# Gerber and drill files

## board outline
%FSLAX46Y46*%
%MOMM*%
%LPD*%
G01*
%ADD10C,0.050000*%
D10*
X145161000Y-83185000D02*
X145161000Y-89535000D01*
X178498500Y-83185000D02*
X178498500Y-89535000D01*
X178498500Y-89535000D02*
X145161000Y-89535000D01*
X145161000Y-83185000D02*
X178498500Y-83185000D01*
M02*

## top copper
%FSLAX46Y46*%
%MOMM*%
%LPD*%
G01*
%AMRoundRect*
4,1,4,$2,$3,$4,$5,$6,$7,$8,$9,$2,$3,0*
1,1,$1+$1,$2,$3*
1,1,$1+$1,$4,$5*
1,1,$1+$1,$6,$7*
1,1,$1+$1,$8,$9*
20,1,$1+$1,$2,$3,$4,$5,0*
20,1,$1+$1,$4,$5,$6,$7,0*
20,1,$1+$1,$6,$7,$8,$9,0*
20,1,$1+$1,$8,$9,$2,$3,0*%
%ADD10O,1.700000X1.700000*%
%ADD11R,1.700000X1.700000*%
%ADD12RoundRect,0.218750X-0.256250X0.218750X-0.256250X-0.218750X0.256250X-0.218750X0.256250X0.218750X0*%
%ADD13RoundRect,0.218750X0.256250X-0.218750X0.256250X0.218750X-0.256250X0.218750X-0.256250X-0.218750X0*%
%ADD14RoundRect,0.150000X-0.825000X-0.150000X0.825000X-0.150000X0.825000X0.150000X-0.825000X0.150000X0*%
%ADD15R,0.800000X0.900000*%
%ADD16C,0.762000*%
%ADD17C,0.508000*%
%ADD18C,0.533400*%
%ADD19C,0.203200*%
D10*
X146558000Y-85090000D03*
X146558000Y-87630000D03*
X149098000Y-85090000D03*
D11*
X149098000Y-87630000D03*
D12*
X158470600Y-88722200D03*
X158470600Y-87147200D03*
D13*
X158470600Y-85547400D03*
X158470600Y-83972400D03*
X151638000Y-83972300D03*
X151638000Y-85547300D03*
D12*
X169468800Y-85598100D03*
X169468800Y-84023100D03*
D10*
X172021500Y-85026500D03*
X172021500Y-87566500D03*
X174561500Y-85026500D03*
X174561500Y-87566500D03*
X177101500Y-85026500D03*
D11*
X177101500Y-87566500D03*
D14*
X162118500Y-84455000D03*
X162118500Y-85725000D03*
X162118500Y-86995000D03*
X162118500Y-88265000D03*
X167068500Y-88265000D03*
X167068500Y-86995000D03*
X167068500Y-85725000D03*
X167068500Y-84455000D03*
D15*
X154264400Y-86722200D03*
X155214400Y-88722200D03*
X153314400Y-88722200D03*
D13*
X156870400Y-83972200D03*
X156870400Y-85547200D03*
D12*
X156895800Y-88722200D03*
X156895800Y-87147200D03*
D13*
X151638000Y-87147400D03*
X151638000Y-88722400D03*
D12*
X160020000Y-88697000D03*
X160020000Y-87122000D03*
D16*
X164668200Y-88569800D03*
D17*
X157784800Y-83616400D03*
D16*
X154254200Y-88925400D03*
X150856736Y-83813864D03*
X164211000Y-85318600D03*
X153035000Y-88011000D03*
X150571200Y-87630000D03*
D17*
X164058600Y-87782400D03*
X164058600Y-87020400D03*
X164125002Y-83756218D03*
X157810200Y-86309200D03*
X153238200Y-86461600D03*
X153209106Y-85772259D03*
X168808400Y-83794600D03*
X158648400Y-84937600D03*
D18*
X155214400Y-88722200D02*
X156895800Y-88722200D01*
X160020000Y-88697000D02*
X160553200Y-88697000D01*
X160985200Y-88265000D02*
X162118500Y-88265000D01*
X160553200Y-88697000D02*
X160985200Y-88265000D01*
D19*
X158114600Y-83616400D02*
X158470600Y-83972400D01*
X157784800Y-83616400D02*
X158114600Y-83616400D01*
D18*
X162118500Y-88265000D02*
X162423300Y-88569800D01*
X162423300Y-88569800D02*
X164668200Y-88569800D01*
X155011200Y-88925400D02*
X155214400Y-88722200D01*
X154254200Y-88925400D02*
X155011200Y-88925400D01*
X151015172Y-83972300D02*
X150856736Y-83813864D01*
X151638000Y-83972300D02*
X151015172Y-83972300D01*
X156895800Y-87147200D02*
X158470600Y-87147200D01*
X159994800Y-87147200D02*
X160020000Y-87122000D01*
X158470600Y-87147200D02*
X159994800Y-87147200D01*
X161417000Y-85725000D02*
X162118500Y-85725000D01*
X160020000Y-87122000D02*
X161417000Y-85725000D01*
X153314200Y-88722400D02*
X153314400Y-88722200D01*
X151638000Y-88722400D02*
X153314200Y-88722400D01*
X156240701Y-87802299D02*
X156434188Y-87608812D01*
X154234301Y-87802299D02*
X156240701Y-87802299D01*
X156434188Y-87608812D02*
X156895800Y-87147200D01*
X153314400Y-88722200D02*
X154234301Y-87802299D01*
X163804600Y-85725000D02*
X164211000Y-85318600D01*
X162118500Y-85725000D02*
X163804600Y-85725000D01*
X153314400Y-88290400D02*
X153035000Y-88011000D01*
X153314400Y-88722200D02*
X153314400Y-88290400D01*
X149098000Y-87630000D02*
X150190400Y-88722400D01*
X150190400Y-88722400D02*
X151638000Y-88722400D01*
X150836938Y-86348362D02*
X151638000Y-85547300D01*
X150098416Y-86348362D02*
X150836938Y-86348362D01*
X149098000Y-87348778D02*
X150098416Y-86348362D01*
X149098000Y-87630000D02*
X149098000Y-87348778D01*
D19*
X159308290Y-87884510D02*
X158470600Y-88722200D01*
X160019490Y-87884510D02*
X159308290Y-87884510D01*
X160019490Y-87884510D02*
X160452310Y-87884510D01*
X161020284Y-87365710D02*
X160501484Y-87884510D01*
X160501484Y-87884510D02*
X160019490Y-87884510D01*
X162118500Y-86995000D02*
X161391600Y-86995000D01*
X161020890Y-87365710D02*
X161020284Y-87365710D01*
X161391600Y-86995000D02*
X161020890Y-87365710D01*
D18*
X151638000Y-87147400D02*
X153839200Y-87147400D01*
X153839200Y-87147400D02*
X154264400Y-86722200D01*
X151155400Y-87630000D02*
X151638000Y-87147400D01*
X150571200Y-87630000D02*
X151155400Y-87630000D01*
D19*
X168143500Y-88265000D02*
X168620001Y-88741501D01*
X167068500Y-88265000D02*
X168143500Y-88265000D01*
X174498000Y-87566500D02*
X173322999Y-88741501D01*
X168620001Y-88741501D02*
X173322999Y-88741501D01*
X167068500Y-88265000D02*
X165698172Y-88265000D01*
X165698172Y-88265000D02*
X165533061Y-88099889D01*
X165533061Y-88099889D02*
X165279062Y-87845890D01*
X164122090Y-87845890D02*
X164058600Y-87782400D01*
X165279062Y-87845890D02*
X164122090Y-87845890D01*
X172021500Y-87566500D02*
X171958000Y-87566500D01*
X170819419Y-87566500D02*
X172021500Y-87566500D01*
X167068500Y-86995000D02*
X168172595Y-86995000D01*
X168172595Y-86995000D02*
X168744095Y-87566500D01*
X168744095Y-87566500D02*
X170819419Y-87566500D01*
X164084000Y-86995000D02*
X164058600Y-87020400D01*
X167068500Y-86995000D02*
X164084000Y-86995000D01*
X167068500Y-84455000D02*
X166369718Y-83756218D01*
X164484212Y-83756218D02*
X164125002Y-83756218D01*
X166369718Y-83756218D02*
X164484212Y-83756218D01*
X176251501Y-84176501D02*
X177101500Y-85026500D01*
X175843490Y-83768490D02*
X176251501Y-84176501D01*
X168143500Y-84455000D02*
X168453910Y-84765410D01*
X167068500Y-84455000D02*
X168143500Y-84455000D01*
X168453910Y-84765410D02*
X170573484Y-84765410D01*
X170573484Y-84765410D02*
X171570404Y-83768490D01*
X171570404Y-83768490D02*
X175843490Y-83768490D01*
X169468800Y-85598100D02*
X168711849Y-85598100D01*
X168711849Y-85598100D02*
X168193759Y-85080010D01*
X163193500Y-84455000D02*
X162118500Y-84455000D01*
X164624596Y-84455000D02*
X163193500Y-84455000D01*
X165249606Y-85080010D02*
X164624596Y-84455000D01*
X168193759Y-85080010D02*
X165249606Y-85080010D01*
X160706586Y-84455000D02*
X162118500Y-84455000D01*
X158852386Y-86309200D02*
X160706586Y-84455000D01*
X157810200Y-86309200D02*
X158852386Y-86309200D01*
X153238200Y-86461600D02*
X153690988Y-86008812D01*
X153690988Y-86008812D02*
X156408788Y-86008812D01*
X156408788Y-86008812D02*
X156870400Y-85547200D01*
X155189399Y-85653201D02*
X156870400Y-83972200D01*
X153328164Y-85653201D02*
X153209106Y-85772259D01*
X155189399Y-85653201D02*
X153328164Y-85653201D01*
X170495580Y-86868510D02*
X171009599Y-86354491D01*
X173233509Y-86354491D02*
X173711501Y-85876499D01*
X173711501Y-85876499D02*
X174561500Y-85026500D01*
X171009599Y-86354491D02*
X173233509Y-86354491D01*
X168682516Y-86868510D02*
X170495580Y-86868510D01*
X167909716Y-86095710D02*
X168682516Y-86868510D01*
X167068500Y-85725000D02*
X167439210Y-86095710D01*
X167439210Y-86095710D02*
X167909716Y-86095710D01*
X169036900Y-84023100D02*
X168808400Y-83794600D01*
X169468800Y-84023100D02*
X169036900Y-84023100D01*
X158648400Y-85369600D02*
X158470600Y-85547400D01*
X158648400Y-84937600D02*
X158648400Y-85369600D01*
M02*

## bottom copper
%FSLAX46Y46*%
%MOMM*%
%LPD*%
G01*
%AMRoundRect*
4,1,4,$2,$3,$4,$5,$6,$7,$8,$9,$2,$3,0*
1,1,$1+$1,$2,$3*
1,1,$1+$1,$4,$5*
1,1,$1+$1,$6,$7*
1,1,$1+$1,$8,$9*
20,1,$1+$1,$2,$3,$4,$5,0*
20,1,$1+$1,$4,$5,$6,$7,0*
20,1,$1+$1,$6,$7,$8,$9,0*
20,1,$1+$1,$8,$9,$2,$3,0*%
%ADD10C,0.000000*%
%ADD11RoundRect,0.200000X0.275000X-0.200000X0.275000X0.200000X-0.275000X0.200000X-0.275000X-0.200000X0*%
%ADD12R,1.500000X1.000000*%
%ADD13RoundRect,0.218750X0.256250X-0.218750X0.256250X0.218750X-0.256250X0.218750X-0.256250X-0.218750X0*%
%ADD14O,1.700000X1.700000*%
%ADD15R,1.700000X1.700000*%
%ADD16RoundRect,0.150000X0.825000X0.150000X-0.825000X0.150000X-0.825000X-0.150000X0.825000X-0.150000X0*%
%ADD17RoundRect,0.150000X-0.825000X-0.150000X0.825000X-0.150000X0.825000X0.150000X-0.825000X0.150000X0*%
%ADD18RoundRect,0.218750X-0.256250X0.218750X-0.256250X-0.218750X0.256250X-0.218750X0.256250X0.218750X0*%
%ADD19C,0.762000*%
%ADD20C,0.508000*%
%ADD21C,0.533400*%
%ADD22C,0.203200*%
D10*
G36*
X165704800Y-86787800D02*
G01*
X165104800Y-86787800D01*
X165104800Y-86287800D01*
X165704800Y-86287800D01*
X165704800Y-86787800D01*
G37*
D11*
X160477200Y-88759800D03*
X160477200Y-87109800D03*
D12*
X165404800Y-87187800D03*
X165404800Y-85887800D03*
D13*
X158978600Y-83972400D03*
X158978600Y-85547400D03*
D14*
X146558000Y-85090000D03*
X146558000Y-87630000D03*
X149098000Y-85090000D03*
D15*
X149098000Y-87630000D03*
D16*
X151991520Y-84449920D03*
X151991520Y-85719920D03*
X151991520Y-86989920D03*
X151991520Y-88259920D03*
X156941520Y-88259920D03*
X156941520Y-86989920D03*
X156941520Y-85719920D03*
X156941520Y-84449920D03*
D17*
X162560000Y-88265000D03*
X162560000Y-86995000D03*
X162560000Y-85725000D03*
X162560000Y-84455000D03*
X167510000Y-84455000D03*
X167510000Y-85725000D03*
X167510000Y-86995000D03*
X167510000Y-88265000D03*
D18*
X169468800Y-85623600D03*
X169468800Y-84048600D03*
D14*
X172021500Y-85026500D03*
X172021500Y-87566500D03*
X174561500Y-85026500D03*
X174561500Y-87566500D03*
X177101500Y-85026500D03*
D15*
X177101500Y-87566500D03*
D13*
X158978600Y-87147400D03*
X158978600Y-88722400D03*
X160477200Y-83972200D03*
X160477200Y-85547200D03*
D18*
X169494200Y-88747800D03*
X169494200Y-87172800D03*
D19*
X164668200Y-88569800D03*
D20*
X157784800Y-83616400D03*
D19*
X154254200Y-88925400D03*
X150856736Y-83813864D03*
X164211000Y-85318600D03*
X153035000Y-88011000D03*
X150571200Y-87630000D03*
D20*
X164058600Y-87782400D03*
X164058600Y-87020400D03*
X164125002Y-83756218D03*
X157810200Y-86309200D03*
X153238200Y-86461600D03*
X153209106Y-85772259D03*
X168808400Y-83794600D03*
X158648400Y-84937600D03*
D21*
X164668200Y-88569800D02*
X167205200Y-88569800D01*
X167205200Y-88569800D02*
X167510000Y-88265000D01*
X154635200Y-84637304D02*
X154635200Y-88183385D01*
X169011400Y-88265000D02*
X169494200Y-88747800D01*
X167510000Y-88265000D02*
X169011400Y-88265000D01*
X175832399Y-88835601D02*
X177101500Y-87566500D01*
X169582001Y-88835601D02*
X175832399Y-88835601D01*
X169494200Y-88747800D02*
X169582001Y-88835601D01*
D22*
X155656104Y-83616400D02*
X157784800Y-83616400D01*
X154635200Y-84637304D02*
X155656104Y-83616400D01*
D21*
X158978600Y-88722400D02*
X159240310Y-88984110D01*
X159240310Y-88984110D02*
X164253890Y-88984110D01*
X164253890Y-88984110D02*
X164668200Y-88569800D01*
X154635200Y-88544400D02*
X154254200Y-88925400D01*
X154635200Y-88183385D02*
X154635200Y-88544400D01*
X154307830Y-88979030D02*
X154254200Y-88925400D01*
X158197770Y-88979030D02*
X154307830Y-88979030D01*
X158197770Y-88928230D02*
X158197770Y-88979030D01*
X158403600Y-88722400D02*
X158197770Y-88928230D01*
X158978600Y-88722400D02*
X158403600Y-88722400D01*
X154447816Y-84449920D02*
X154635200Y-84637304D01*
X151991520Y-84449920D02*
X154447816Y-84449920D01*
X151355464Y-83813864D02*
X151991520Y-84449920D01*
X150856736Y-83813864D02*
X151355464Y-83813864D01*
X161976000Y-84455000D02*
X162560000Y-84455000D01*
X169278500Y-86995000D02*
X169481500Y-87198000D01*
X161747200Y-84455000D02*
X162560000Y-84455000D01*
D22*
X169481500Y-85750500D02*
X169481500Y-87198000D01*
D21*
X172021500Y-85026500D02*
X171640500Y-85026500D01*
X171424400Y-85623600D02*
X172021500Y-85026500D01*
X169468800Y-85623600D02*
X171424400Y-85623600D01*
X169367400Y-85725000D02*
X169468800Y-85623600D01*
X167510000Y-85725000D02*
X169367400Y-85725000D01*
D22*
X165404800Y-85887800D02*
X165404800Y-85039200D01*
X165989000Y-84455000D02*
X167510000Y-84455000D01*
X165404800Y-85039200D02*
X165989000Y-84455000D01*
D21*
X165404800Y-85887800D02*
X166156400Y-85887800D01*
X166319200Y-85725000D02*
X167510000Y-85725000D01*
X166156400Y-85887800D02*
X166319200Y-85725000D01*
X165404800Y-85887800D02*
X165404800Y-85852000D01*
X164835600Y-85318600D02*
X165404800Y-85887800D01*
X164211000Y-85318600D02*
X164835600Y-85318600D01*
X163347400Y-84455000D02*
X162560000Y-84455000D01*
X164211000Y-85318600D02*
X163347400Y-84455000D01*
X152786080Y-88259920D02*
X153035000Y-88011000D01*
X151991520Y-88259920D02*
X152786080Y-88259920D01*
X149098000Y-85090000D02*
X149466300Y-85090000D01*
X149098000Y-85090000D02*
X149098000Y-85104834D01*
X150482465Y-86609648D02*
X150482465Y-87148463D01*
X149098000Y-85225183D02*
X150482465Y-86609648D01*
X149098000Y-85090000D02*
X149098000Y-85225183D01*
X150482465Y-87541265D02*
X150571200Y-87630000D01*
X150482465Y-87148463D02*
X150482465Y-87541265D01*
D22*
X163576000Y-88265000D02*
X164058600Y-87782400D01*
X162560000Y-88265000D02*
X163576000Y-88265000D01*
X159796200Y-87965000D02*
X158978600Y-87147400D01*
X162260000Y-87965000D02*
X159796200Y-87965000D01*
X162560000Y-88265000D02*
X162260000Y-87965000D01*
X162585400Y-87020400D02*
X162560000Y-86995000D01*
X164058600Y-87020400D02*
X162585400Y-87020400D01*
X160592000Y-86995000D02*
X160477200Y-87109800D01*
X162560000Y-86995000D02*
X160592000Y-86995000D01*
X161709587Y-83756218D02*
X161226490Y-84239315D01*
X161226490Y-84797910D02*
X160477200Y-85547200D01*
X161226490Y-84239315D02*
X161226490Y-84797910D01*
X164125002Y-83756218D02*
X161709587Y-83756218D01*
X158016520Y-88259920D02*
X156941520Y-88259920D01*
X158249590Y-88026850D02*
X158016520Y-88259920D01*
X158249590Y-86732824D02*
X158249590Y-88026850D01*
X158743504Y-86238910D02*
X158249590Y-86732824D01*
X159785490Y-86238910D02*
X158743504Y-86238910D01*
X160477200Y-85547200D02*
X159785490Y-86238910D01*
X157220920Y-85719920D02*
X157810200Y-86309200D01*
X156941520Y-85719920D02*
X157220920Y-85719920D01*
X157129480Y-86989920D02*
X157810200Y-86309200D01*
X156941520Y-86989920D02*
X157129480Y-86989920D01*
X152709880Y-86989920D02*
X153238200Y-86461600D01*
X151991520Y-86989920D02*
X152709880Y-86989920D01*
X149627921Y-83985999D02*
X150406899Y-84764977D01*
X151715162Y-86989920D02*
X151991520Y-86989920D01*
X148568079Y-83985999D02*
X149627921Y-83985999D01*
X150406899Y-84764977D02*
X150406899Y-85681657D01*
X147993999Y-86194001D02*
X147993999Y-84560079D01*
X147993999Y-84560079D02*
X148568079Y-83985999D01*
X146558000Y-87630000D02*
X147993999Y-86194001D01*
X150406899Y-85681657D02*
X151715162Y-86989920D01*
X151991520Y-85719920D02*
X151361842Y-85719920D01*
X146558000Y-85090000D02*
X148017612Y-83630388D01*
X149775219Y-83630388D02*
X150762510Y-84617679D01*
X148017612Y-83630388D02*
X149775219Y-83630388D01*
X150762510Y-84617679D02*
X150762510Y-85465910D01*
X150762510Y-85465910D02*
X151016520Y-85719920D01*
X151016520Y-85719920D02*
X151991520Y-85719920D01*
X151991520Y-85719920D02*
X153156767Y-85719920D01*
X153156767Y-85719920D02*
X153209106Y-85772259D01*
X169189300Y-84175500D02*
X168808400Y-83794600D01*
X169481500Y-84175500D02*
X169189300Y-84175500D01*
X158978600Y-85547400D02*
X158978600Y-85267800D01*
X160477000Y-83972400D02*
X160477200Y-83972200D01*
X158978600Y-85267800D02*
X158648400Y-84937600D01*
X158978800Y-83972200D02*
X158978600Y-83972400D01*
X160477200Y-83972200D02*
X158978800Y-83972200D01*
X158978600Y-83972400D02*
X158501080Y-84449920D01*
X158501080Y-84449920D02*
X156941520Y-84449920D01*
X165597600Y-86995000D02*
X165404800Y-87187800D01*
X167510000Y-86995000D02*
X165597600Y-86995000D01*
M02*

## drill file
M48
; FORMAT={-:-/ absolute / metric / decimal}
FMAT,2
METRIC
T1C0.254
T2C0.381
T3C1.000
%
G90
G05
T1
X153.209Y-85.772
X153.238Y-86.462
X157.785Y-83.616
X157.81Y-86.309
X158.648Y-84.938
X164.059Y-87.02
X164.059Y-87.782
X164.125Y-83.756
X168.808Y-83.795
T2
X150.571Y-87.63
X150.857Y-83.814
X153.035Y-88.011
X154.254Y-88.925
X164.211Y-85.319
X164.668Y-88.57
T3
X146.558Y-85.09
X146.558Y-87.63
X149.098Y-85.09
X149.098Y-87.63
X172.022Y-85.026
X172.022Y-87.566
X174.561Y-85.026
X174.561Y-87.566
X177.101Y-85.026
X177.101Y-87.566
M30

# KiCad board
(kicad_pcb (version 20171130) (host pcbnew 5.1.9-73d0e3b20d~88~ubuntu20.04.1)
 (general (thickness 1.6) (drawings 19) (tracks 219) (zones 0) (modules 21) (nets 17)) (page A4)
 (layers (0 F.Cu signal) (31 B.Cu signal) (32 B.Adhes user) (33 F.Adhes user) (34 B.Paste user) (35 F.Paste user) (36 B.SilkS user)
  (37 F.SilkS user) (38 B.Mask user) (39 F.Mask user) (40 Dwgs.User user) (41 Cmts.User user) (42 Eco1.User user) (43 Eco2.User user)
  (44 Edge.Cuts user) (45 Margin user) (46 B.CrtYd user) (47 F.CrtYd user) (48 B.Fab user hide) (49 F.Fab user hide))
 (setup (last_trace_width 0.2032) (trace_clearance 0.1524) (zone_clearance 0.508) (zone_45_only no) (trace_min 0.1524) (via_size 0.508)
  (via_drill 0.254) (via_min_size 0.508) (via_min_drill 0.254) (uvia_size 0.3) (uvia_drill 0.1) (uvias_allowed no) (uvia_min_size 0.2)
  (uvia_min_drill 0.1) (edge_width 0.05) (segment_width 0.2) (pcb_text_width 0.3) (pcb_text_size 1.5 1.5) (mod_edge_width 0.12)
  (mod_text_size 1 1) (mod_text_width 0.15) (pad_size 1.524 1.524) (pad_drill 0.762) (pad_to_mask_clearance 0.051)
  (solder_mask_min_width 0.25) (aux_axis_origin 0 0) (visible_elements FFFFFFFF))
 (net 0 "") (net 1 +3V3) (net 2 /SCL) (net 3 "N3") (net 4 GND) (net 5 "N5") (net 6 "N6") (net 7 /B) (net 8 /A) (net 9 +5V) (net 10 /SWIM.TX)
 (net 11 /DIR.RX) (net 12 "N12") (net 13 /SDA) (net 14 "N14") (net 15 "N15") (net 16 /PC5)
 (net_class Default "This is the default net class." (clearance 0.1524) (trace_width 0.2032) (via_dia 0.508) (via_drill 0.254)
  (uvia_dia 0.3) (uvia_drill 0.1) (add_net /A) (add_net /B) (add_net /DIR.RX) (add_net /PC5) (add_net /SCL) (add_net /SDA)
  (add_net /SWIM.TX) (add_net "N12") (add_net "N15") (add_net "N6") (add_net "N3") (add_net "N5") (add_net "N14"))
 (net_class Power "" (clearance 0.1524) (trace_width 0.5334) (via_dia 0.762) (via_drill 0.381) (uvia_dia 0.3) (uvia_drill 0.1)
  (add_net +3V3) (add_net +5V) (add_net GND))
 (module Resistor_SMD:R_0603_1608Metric (layer B.Cu) (at 160.4772 87.9348 90)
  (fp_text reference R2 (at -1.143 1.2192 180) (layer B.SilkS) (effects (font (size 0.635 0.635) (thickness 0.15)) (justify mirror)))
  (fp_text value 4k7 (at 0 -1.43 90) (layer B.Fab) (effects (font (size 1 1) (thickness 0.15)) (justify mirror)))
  (pad 1 smd roundrect (at -0.825 0 90) (size 0.8 0.95) (layers B.Cu B.Paste B.Mask) (roundrect_rratio 0.25) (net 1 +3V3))
  (pad 2 smd roundrect (at 0.825 0 90) (size 0.8 0.95) (layers B.Cu B.Paste B.Mask) (roundrect_rratio 0.25) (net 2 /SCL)))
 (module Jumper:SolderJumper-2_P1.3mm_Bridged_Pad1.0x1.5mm (layer B.Cu) (at 165.4048 86.5378 270)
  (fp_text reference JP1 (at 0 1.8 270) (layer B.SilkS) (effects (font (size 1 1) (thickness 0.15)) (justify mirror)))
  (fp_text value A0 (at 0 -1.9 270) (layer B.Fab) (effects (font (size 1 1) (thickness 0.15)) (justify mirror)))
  (fp_poly (pts (xy -0.25 0.3) (xy 0.25 0.3) (xy 0.25 -0.3) (xy -0.25 -0.3)) (layer B.Cu) (width 0))
  (pad 2 smd rect (at 0.65 0 270) (size 1 1.5) (layers B.Cu B.Mask) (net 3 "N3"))
  (pad 1 smd rect (at -0.65 0 270) (size 1 1.5) (layers B.Cu B.Mask) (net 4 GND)))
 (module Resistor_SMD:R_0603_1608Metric (layer B.Cu) (at 158.9786 84.7599 90)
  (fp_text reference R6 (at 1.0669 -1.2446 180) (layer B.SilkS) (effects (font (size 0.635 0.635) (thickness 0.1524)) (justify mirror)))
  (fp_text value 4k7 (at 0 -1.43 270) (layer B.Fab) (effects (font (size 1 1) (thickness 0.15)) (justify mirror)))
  (pad 2 smd roundrect (at 0.7875 0 90) (size 0.875 0.95) (layers B.Cu B.Paste B.Mask) (roundrect_rratio 0.25) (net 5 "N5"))
  (pad 1 smd roundrect (at -0.7875 0 90) (size 0.875 0.95) (layers B.Cu B.Paste B.Mask) (roundrect_rratio 0.25) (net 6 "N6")))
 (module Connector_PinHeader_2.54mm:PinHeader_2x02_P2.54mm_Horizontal (layer B.Cu) (at 149.098 87.63 90)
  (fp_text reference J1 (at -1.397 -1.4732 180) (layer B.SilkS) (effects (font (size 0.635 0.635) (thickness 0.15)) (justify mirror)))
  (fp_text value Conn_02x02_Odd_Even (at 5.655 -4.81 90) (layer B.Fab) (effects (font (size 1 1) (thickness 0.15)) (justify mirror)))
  (pad 4 thru_hole oval (at 2.54 -2.54 90) (size 1.7 1.7) (drill 1) (layers *.Cu *.Mask) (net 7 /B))
  (pad 3 thru_hole oval (at 0 -2.54 90) (size 1.7 1.7) (drill 1) (layers *.Cu *.Mask) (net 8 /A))
  (pad 2 thru_hole oval (at 2.54 0 90) (size 1.7 1.7) (drill 1) (layers *.Cu *.Mask) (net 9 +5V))
  (pad 1 thru_hole rect (at 0 0 90) (size 1.7 1.7) (drill 1) (layers *.Cu *.Mask) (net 4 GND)))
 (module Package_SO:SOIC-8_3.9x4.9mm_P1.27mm (layer B.Cu) (at 154.46652 86.35492 180)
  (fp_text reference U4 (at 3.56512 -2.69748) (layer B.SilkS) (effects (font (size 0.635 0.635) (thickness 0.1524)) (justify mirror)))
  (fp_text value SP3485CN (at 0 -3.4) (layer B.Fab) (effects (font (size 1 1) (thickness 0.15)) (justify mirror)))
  (pad 8 smd roundrect (at 2.475 1.905 180) (size 1.95 0.6) (layers B.Cu B.Paste B.Mask) (roundrect_rratio 0.25) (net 1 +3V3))
  (pad 7 smd roundrect (at 2.475 0.635 180) (size 1.95 0.6) (layers B.Cu B.Paste B.Mask) (roundrect_rratio 0.25) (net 7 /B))
  (pad 6 smd roundrect (at 2.475 -0.635 180) (size 1.95 0.6) (layers B.Cu B.Paste B.Mask) (roundrect_rratio 0.25) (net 8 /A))
  (pad 5 smd roundrect (at 2.475 -1.905 180) (size 1.95 0.6) (layers B.Cu B.Paste B.Mask) (roundrect_rratio 0.25) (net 4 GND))
  (pad 4 smd roundrect (at -2.475 -1.905 180) (size 1.95 0.6) (layers B.Cu B.Paste B.Mask) (roundrect_rratio 0.25) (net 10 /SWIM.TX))
  (pad 3 smd roundrect (at -2.475 -0.635 180) (size 1.95 0.6) (layers B.Cu B.Paste B.Mask) (roundrect_rratio 0.25) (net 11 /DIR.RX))
  (pad 2 smd roundrect (at -2.475 0.635 180) (size 1.95 0.6) (layers B.Cu B.Paste B.Mask) (roundrect_rratio 0.25) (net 11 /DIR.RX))
  (pad 1 smd roundrect (at -2.475 1.905 180) (size 1.95 0.6) (layers B.Cu B.Paste B.Mask) (roundrect_rratio 0.25) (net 5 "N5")))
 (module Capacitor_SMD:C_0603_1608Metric (layer F.Cu) (at 158.4706 87.9347 270)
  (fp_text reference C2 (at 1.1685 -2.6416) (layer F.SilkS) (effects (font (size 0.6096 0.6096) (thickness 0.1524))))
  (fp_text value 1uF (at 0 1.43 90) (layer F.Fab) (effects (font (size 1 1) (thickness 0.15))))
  (pad 2 smd roundrect (at 0.7875 0 270) (size 0.875 0.95) (layers F.Cu F.Paste F.Mask) (roundrect_rratio 0.25) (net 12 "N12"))
  (pad 1 smd roundrect (at -0.7875 0 270) (size 0.875 0.95) (layers F.Cu F.Paste F.Mask) (roundrect_rratio 0.25) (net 4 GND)))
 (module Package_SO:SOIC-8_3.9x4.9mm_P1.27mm (layer B.Cu) (at 165.035 86.36)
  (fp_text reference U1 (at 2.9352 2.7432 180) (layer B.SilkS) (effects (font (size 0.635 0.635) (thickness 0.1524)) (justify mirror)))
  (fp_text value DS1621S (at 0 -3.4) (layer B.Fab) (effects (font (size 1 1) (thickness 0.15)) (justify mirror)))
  (pad 1 smd roundrect (at -2.475 1.905) (size 1.95 0.6) (layers B.Cu B.Paste B.Mask) (roundrect_rratio 0.25) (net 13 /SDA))
  (pad 2 smd roundrect (at -2.475 0.635) (size 1.95 0.6) (layers B.Cu B.Paste B.Mask) (roundrect_rratio 0.25) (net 2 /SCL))
  (pad 3 smd roundrect (at -2.475 -0.635) (size 1.95 0.6) (layers B.Cu B.Paste B.Mask) (roundrect_rratio 0.25) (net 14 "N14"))
  (pad 4 smd roundrect (at -2.475 -1.905) (size 1.95 0.6) (layers B.Cu B.Paste B.Mask) (roundrect_rratio 0.25) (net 4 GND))
  (pad 5 smd roundrect (at 2.475 -1.905) (size 1.95 0.6) (layers B.Cu B.Paste B.Mask) (roundrect_rratio 0.25) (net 4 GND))
  (pad 6 smd roundrect (at 2.475 -0.635) (size 1.95 0.6) (layers B.Cu B.Paste B.Mask) (roundrect_rratio 0.25) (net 4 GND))
  (pad 7 smd roundrect (at 2.475 0.635) (size 1.95 0.6) (layers B.Cu B.Paste B.Mask) (roundrect_rratio 0.25) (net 3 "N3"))
  (pad 8 smd roundrect (at 2.475 1.905) (size 1.95 0.6) (layers B.Cu B.Paste B.Mask) (roundrect_rratio 0.25) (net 1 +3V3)))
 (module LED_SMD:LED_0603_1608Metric (layer F.Cu) (at 158.4706 84.7599 90)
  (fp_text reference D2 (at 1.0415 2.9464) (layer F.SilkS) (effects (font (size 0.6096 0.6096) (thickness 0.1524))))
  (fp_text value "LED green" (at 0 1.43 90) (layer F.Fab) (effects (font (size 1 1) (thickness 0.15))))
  (pad 1 smd roundrect (at -0.7875 0 90) (size 0.875 0.95) (layers F.Cu F.Paste F.Mask) (roundrect_rratio 0.25) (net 6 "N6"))
  (pad 2 smd roundrect (at 0.7875 0 90) (size 0.875 0.95) (layers F.Cu F.Paste F.Mask) (roundrect_rratio 0.25) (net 1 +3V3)))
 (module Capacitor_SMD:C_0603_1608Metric (layer F.Cu) (at 151.638 84.7598 90)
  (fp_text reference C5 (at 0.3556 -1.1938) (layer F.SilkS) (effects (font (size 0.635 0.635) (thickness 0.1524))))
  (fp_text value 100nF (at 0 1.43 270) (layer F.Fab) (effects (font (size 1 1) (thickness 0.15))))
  (pad 2 smd roundrect (at 0.7875 0 90) (size 0.875 0.95) (layers F.Cu F.Paste F.Mask) (roundrect_rratio 0.25) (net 1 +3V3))
  (pad 1 smd roundrect (at -0.7875 0 90) (size 0.875 0.95) (layers F.Cu F.Paste F.Mask) (roundrect_rratio 0.25) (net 4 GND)))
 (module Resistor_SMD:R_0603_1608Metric (layer B.Cu) (at 169.4688 84.8361 270)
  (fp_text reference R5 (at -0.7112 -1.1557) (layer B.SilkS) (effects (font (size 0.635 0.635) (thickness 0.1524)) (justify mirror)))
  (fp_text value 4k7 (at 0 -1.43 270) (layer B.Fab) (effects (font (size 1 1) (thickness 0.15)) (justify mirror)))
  (pad 2 smd roundrect (at 0.7875 0 270) (size 0.875 0.95) (layers B.Cu B.Paste B.Mask) (roundrect_rratio 0.25) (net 4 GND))
  (pad 1 smd roundrect (at -0.7875 0 270) (size 0.875 0.95) (layers B.Cu B.Paste B.Mask) (roundrect_rratio 0.25) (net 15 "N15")))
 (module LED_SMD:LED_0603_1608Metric (layer F.Cu) (at 169.4688 84.8106 270)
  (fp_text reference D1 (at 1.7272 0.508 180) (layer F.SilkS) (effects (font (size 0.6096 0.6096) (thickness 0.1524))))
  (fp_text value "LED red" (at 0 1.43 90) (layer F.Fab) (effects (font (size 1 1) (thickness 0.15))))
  (pad 2 smd roundrect (at 0.7875 0 270) (size 0.875 0.95) (layers F.Cu F.Paste F.Mask) (roundrect_rratio 0.25) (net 11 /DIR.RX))
  (pad 1 smd roundrect (at -0.7875 0 270) (size 0.875 0.95) (layers F.Cu F.Paste F.Mask) (roundrect_rratio 0.25) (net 15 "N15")))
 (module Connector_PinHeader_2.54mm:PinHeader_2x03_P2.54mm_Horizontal (layer B.Cu) (at 177.1015 87.5665 90)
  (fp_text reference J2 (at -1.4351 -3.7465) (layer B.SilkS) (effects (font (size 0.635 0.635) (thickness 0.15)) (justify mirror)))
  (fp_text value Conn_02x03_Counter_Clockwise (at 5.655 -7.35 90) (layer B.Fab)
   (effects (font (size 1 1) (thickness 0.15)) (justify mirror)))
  (pad 6 thru_hole oval (at 2.54 -5.08 90) (size 1.7 1.7) (drill 1) (layers *.Cu *.Mask) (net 4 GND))
  (pad 5 thru_hole oval (at 0 -5.08 90) (size 1.7 1.7) (drill 1) (layers *.Cu *.Mask) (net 2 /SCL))
  (pad 4 thru_hole oval (at 2.54 -2.54 90) (size 1.7 1.7) (drill 1) (layers *.Cu *.Mask) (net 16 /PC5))
  (pad 3 thru_hole oval (at 0 -2.54 90) (size 1.7 1.7) (drill 1) (layers *.Cu *.Mask) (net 13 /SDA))
  (pad 2 thru_hole oval (at 2.54 0 90) (size 1.7 1.7) (drill 1) (layers *.Cu *.Mask) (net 10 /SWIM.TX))
  (pad 1 thru_hole rect (at 0 0 90) (size 1.7 1.7) (drill 1) (layers *.Cu *.Mask) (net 1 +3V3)))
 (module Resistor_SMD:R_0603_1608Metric (layer B.Cu) (at 158.9786 87.9349 90)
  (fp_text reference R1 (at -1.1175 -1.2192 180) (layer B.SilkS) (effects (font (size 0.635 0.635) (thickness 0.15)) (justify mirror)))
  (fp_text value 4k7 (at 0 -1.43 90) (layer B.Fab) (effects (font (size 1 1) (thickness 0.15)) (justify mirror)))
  (pad 2 smd roundrect (at 0.7875 0 90) (size 0.875 0.95) (layers B.Cu B.Paste B.Mask) (roundrect_rratio 0.25) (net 13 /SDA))
  (pad 1 smd roundrect (at -0.7875 0 90) (size 0.875 0.95) (layers B.Cu B.Paste B.Mask) (roundrect_rratio 0.25) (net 1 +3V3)))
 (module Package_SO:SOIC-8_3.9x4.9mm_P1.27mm (layer F.Cu) (at 164.5935 86.36)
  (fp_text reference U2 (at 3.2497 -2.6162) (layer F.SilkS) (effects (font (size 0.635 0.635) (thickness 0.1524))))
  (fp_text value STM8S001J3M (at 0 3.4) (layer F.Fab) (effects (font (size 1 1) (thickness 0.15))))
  (pad 1 smd roundrect (at -2.475 -1.905) (size 1.95 0.6) (layers F.Cu F.Paste F.Mask) (roundrect_rratio 0.25) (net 11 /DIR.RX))
  (pad 2 smd roundrect (at -2.475 -0.635) (size 1.95 0.6) (layers F.Cu F.Paste F.Mask) (roundrect_rratio 0.25) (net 4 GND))
  (pad 3 smd roundrect (at -2.475 0.635) (size 1.95 0.6) (layers F.Cu F.Paste F.Mask) (roundrect_rratio 0.25) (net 12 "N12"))
  (pad 4 smd roundrect (at -2.475 1.905) (size 1.95 0.6) (layers F.Cu F.Paste F.Mask) (roundrect_rratio 0.25) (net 1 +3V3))
  (pad 5 smd roundrect (at 2.475 1.905) (size 1.95 0.6) (layers F.Cu F.Paste F.Mask) (roundrect_rratio 0.25) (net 13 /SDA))
  (pad 6 smd roundrect (at 2.475 0.635) (size 1.95 0.6) (layers F.Cu F.Paste F.Mask) (roundrect_rratio 0.25) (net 2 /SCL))
  (pad 7 smd roundrect (at 2.475 -0.635) (size 1.95 0.6) (layers F.Cu F.Paste F.Mask) (roundrect_rratio 0.25) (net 16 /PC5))
  (pad 8 smd roundrect (at 2.475 -1.905) (size 1.95 0.6) (layers F.Cu F.Paste F.Mask) (roundrect_rratio 0.25) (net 10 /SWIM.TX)))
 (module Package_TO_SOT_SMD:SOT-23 (layer F.Cu) (at 154.2644 87.7222 90)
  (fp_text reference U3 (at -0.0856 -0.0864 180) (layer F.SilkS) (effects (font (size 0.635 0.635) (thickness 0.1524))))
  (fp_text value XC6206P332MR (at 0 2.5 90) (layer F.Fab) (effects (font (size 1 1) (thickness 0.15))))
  (pad 3 smd rect (at 1 0 90) (size 0.9 0.8) (layers F.Cu F.Paste F.Mask) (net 9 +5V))
  (pad 2 smd rect (at -1 0.95 90) (size 0.9 0.8) (layers F.Cu F.Paste F.Mask) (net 1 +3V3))
  (pad 1 smd rect (at -1 -0.95 90) (size 0.9 0.8) (layers F.Cu F.Paste F.Mask) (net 4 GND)))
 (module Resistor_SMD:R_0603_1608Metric (layer F.Cu) (at 156.8704 84.7597 90)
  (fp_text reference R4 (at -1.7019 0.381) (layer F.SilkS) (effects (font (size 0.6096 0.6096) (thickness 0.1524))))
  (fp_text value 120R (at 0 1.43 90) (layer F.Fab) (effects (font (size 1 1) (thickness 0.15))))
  (pad 2 smd roundrect (at 0.7875 0 90) (size 0.875 0.95) (layers F.Cu F.Paste F.Mask) (roundrect_rratio 0.25) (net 7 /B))
  (pad 1 smd roundrect (at -0.7875 0 90) (size 0.875 0.95) (layers F.Cu F.Paste F.Mask) (roundrect_rratio 0.25) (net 8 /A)))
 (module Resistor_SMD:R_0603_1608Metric (layer B.Cu) (at 160.4772 84.7597 90)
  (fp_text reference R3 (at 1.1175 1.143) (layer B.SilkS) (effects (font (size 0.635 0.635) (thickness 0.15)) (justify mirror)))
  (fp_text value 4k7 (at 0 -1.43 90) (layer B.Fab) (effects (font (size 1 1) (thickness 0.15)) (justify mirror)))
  (pad 2 smd roundrect (at 0.7875 0 90) (size 0.875 0.95) (layers B.Cu B.Paste B.Mask) (roundrect_rratio 0.25) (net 5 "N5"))
  (pad 1 smd roundrect (at -0.7875 0 90) (size 0.875 0.95) (layers B.Cu B.Paste B.Mask) (roundrect_rratio 0.25) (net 10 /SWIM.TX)))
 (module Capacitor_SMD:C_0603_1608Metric (layer F.Cu) (at 156.8958 87.9347 270)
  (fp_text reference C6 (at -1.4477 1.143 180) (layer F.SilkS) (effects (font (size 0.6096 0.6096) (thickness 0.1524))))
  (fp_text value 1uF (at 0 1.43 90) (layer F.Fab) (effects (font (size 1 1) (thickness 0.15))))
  (pad 2 smd roundrect (at 0.7875 0 270) (size 0.875 0.95) (layers F.Cu F.Paste F.Mask) (roundrect_rratio 0.25) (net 1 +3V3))
  (pad 1 smd roundrect (at -0.7875 0 270) (size 0.875 0.95) (layers F.Cu F.Paste F.Mask) (roundrect_rratio 0.25) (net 4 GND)))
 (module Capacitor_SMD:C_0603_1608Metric (layer F.Cu) (at 151.638 87.9349 90)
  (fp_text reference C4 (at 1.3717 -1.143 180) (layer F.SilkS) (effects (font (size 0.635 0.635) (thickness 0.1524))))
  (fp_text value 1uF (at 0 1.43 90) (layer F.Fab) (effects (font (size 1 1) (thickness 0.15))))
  (pad 2 smd roundrect (at 0.7875 0 90) (size 0.875 0.95) (layers F.Cu F.Paste F.Mask) (roundrect_rratio 0.25) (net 9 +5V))
  (pad 1 smd roundrect (at -0.7875 0 90) (size 0.875 0.95) (layers F.Cu F.Paste F.Mask) (roundrect_rratio 0.25) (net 4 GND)))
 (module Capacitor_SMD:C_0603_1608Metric (layer F.Cu) (at 160.02 87.9095 270)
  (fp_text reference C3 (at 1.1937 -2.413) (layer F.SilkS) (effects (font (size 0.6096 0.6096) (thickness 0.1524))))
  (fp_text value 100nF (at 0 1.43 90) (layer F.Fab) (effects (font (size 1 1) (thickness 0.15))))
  (pad 2 smd roundrect (at 0.7875 0 270) (size 0.875 0.95) (layers F.Cu F.Paste F.Mask) (roundrect_rratio 0.25) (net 1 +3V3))
  (pad 1 smd roundrect (at -0.7875 0 270) (size 0.875 0.95) (layers F.Cu F.Paste F.Mask) (roundrect_rratio 0.25) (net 4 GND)))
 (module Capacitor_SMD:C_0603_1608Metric (layer B.Cu) (at 169.4942 87.9603 270)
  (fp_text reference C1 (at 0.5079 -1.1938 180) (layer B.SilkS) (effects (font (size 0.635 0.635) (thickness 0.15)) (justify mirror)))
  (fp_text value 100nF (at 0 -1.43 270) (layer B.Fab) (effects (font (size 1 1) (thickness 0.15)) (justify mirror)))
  (pad 2 smd roundrect (at 0.7875 0 270) (size 0.875 0.95) (layers B.Cu B.Paste B.Mask) (roundrect_rratio 0.25) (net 1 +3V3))
  (pad 1 smd roundrect (at -0.7875 0 270) (size 0.875 0.95) (layers B.Cu B.Paste B.Mask) (roundrect_rratio 0.25) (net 4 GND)))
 (gr_line (start 145.161 83.185) (end 145.161 89.535) (layer Edge.Cuts) (width 0.05))
 (gr_line (start 178.4985 83.185) (end 178.4985 89.535) (layer Edge.Cuts) (width 0.05))
 (gr_line (start 178.4985 89.535) (end 145.161 89.535) (layer Edge.Cuts) (width 0.05))
 (gr_line (start 145.161 83.185) (end 178.4985 83.185) (layer Edge.Cuts) (width 0.05))
 (via (at 164.6682 88.5698) (size 0.762) (drill 0.381) (layers F.Cu B.Cu) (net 1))
 (segment (start 164.6682 88.5698) (end 167.2052 88.5698) (width 0.5334) (layer B.Cu) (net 1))
 (segment (start 167.2052 88.5698) (end 167.51 88.265) (width 0.5334) (layer B.Cu) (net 1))
 (segment (start 155.2144 88.7222) (end 156.8958 88.7222) (width 0.5334) (layer F.Cu) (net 1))
 (segment (start 154.6352 84.637304) (end 154.6352 88.183385) (width 0.5334) (layer B.Cu) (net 1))
 (segment (start 169.0114 88.265) (end 169.4942 88.7478) (width 0.5334) (layer B.Cu) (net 1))
 (segment (start 167.51 88.265) (end 169.0114 88.265) (width 0.5334) (layer B.Cu) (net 1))
 (segment (start 175.832399 88.835601) (end 177.1015 87.5665) (width 0.5334) (layer B.Cu) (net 1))
 (segment (start 169.582001 88.835601) (end 175.832399 88.835601) (width 0.5334) (layer B.Cu) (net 1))
 (segment (start 169.4942 88.7478) (end 169.582001 88.835601) (width 0.5334) (layer B.Cu) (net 1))
 (segment (start 160.02 88.697) (end 160.5532 88.697) (width 0.5334) (layer F.Cu) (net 1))
 (segment (start 160.9852 88.265) (end 162.1185 88.265) (width 0.5334) (layer F.Cu) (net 1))
 (segment (start 160.5532 88.697) (end 160.9852 88.265) (width 0.5334) (layer F.Cu) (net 1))
 (segment (start 155.656104 83.6164) (end 157.7848 83.6164) (width 0.2032) (layer B.Cu) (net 1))
 (segment (start 154.6352 84.637304) (end 155.656104 83.6164) (width 0.2032) (layer B.Cu) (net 1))
 (via (at 157.7848 83.6164) (size 0.508) (drill 0.254) (layers F.Cu B.Cu) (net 1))
 (segment (start 158.1146 83.6164) (end 158.4706 83.9724) (width 0.2032) (layer F.Cu) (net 1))
 (segment (start 157.7848 83.6164) (end 158.1146 83.6164) (width 0.2032) (layer F.Cu) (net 1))
 (segment (start 162.1185 88.265) (end 162.4233 88.5698) (width 0.5334) (layer F.Cu) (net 1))
 (segment (start 162.4233 88.5698) (end 164.6682 88.5698) (width 0.5334) (layer F.Cu) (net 1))
 (segment (start 158.9786 88.7224) (end 159.24031 88.98411) (width 0.5334) (layer B.Cu) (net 1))
 (segment (start 159.24031 88.98411) (end 164.25389 88.98411) (width 0.5334) (layer B.Cu) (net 1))
 (segment (start 164.25389 88.98411) (end 164.6682 88.5698) (width 0.5334) (layer B.Cu) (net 1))
 (via (at 154.2542 88.9254) (size 0.762) (drill 0.381) (layers F.Cu B.Cu) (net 1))
 (segment (start 154.6352 88.5444) (end 154.2542 88.9254) (width 0.5334) (layer B.Cu) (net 1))
 (segment (start 154.6352 88.183385) (end 154.6352 88.5444) (width 0.5334) (layer B.Cu) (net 1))
 (segment (start 155.0112 88.9254) (end 155.2144 88.7222) (width 0.5334) (layer F.Cu) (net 1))
 (segment (start 154.2542 88.9254) (end 155.0112 88.9254) (width 0.5334) (layer F.Cu) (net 1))
 (segment (start 154.30783 88.97903) (end 154.2542 88.9254) (width 0.5334) (layer B.Cu) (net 1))
 (segment (start 158.19777 88.97903) (end 154.30783 88.97903) (width 0.5334) (layer B.Cu) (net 1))
 (segment (start 158.19777 88.92823) (end 158.19777 88.97903) (width 0.5334) (layer B.Cu) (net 1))
 (segment (start 158.4036 88.7224) (end 158.19777 88.92823) (width 0.5334) (layer B.Cu) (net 1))
 (segment (start 158.9786 88.7224) (end 158.4036 88.7224) (width 0.5334) (layer B.Cu) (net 1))
 (segment (start 154.447816 84.44992) (end 154.6352 84.637304) (width 0.5334) (layer B.Cu) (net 1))
 (segment (start 151.99152 84.44992) (end 154.447816 84.44992) (width 0.5334) (layer B.Cu) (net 1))
 (via (at 150.856736 83.813864) (size 0.762) (drill 0.381) (layers F.Cu B.Cu) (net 1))
 (segment (start 151.015172 83.9723) (end 150.856736 83.813864) (width 0.5334) (layer F.Cu) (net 1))
 (segment (start 151.638 83.9723) (end 151.015172 83.9723) (width 0.5334) (layer F.Cu) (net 1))
 (segment (start 151.355464 83.813864) (end 151.99152 84.44992) (width 0.5334) (layer B.Cu) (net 1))
 (segment (start 150.856736 83.813864) (end 151.355464 83.813864) (width 0.5334) (layer B.Cu) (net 1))
 (segment (start 161.976 84.455) (end 162.56 84.455) (width 0.5334) (layer B.Cu) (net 4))
 (segment (start 156.8958 87.1472) (end 158.4706 87.1472) (width 0.5334) (layer F.Cu) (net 4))
 (segment (start 159.9948 87.1472) (end 160.02 87.122) (width 0.5334) (layer F.Cu) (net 4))
 (segment (start 158.4706 87.1472) (end 159.9948 87.1472) (width 0.5334) (layer F.Cu) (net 4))
 (segment (start 161.417 85.725) (end 162.1185 85.725) (width 0.5334) (layer F.Cu) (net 4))
 (segment (start 160.02 87.122) (end 161.417 85.725) (width 0.5334) (layer F.Cu) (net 4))
 (segment (start 169.2785 86.995) (end 169.4815 87.198) (width 0.5334) (layer B.Cu) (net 4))
 (segment (start 161.7472 84.455) (end 162.56 84.455) (width 0.5334) (layer B.Cu) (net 4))
 (segment (start 169.4815 85.7505) (end 169.4815 87.198) (width 0.2032) (layer B.Cu) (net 4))
 (segment (start 153.3142 88.7224) (end 153.3144 88.7222) (width 0.5334) (layer F.Cu) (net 4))
 (segment (start 151.638 88.7224) (end 153.3142 88.7224) (width 0.5334) (layer F.Cu) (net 4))
 (segment (start 156.240701 87.802299) (end 156.434188 87.608812) (width 0.5334) (layer F.Cu) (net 4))
 (segment (start 154.234301 87.802299) (end 156.240701 87.802299) (width 0.5334) (layer F.Cu) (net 4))
 (segment (start 156.434188 87.608812) (end 156.8958 87.1472) (width 0.5334) (layer F.Cu) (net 4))
 (segment (start 153.3144 88.7222) (end 154.234301 87.802299) (width 0.5334) (layer F.Cu) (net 4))
 (segment (start 172.0215 85.0265) (end 171.6405 85.0265) (width 0.5334) (layer B.Cu) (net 4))
 (segment (start 171.4244 85.6236) (end 172.0215 85.0265) (width 0.5334) (layer B.Cu) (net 4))
 (segment (start 169.4688 85.6236) (end 171.4244 85.6236) (width 0.5334) (layer B.Cu) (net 4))
 (segment (start 169.3674 85.725) (end 169.4688 85.6236) (width 0.5334) (layer B.Cu) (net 4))
 (segment (start 167.51 85.725) (end 169.3674 85.725) (width 0.5334) (layer B.Cu) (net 4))
 (segment (start 165.4048 85.8878) (end 165.4048 85.0392) (width 0.2032) (layer B.Cu) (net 4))
 (segment (start 165.989 84.455) (end 167.51 84.455) (width 0.2032) (layer B.Cu) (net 4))
 (segment (start 165.4048 85.0392) (end 165.989 84.455) (width 0.2032) (layer B.Cu) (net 4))
 (segment (start 165.4048 85.8878) (end 166.1564 85.8878) (width 0.5334) (layer B.Cu) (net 4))
 (segment (start 166.3192 85.725) (end 167.51 85.725) (width 0.5334) (layer B.Cu) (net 4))
 (segment (start 166.1564 85.8878) (end 166.3192 85.725) (width 0.5334) (layer B.Cu) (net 4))
 (segment (start 165.4048 85.8878) (end 165.4048 85.852) (width 0.5334) (layer B.Cu) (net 4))
 (via (at 164.211 85.3186) (size 0.762) (drill 0.381) (layers F.Cu B.Cu) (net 4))
 (segment (start 163.8046 85.725) (end 164.211 85.3186) (width 0.5334) (layer F.Cu) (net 4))
 (segment (start 162.1185 85.725) (end 163.8046 85.725) (width 0.5334) (layer F.Cu) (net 4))
 (segment (start 164.8356 85.3186) (end 165.4048 85.8878) (width 0.5334) (layer B.Cu) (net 4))
 (segment (start 164.211 85.3186) (end 164.8356 85.3186) (width 0.5334) (layer B.Cu) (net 4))
 (segment (start 163.3474 84.455) (end 162.56 84.455) (width 0.5334) (layer B.Cu) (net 4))
 (segment (start 164.211 85.3186) (end 163.3474 84.455) (width 0.5334) (layer B.Cu) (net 4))
 (via (at 153.035 88.011) (size 0.762) (drill 0.381) (layers F.Cu B.Cu) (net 4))
 (segment (start 153.3144 88.2904) (end 153.035 88.011) (width 0.5334) (layer F.Cu) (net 4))
 (segment (start 153.3144 88.7222) (end 153.3144 88.2904) (width 0.5334) (layer F.Cu) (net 4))
 (segment (start 152.78608 88.25992) (end 153.035 88.011) (width 0.5334) (layer B.Cu) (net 4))
 (segment (start 151.99152 88.25992) (end 152.78608 88.25992) (width 0.5334) (layer B.Cu) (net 4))
 (segment (start 149.098 87.63) (end 150.1904 88.7224) (width 0.5334) (layer F.Cu) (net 4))
 (segment (start 150.1904 88.7224) (end 151.638 88.7224) (width 0.5334) (layer F.Cu) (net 4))
 (segment (start 150.836938 86.348362) (end 151.638 85.5473) (width 0.5334) (layer F.Cu) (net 4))
 (segment (start 150.098416 86.348362) (end 150.836938 86.348362) (width 0.5334) (layer F.Cu) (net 4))
 (segment (start 149.098 87.348778) (end 150.098416 86.348362) (width 0.5334) (layer F.Cu) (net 4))
 (segment (start 149.098 87.63) (end 149.098 87.348778) (width 0.5334) (layer F.Cu) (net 4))
 (segment (start 159.30829 87.88451) (end 158.4706 88.7222) (width 0.2032) (layer F.Cu) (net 12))
 (segment (start 160.01949 87.88451) (end 159.30829 87.88451) (width 0.2032) (layer F.Cu) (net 12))
 (segment (start 160.01949 87.88451) (end 160.45231 87.88451) (width 0.2032) (layer F.Cu) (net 12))
 (segment (start 161.020284 87.36571) (end 160.501484 87.88451) (width 0.2032) (layer F.Cu) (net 12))
 (segment (start 160.501484 87.88451) (end 160.01949 87.88451) (width 0.2032) (layer F.Cu) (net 12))
 (segment (start 162.1185 86.995) (end 161.3916 86.995) (width 0.2032) (layer F.Cu) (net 12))
 (segment (start 161.02089 87.36571) (end 161.020284 87.36571) (width 0.2032) (layer F.Cu) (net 12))
 (segment (start 161.3916 86.995) (end 161.02089 87.36571) (width 0.2032) (layer F.Cu) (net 12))
 (segment (start 151.638 87.1474) (end 153.8392 87.1474) (width 0.5334) (layer F.Cu) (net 9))
 (segment (start 153.8392 87.1474) (end 154.2644 86.7222) (width 0.5334) (layer F.Cu) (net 9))
 (segment (start 149.098 85.09) (end 149.4663 85.09) (width 0.5334) (layer B.Cu) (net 9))
 (segment (start 149.098 85.09) (end 149.098 85.104834) (width 0.5334) (layer B.Cu) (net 9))
 (segment (start 150.482465 86.609648) (end 150.482465 87.148463) (width 0.5334) (layer B.Cu) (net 9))
 (segment (start 149.098 85.225183) (end 150.482465 86.609648) (width 0.5334) (layer B.Cu) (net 9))
 (segment (start 149.098 85.09) (end 149.098 85.225183) (width 0.5334) (layer B.Cu) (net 9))
 (via (at 150.5712 87.63) (size 0.762) (drill 0.381) (layers F.Cu B.Cu) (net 9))
 (segment (start 150.482465 87.541265) (end 150.5712 87.63) (width 0.5334) (layer B.Cu) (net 9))
 (segment (start 150.482465 87.148463) (end 150.482465 87.541265) (width 0.5334) (layer B.Cu) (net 9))
 (segment (start 151.1554 87.63) (end 151.638 87.1474) (width 0.5334) (layer F.Cu) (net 9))
 (segment (start 150.5712 87.63) (end 151.1554 87.63) (width 0.5334) (layer F.Cu) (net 9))
 (segment (start 168.1435 88.265) (end 168.620001 88.741501) (width 0.2032) (layer F.Cu) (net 13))
 (segment (start 167.0685 88.265) (end 168.1435 88.265) (width 0.2032) (layer F.Cu) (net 13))
 (segment (start 174.498 87.5665) (end 173.322999 88.741501) (width 0.2032) (layer F.Cu) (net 13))
 (segment (start 168.620001 88.741501) (end 173.322999 88.741501) (width 0.2032) (layer F.Cu) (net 13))
 (segment (start 167.0685 88.265) (end 165.698172 88.265) (width 0.2032) (layer F.Cu) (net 13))
 (segment (start 165.698172 88.265) (end 165.533061 88.099889) (width 0.2032) (layer F.Cu) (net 13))
 (segment (start 165.533061 88.099889) (end 165.279062 87.84589) (width 0.2032) (layer F.Cu) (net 13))
 (via (at 164.0586 87.7824) (size 0.508) (drill 0.254) (layers F.Cu B.Cu) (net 13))
 (segment (start 164.12209 87.84589) (end 164.0586 87.7824) (width 0.2032) (layer F.Cu) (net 13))
 (segment (start 165.279062 87.84589) (end 164.12209 87.84589) (width 0.2032) (layer F.Cu) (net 13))
 (segment (start 163.576 88.265) (end 164.0586 87.7824) (width 0.2032) (layer B.Cu) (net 13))
 (segment (start 162.56 88.265) (end 163.576 88.265) (width 0.2032) (layer B.Cu) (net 13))
 (segment (start 159.7962 87.965) (end 158.9786 87.1474) (width 0.2032) (layer B.Cu) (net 13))
 (segment (start 162.26 87.965) (end 159.7962 87.965) (width 0.2032) (layer B.Cu) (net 13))
 (segment (start 162.56 88.265) (end 162.26 87.965) (width 0.2032) (layer B.Cu) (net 13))
 (segment (start 172.0215 87.5665) (end 171.958 87.5665) (width 0.2032) (layer F.Cu) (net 2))
 (segment (start 170.819419 87.5665) (end 172.0215 87.5665) (width 0.2032) (layer F.Cu) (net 2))
 (segment (start 167.0685 86.995) (end 168.172595 86.995) (width 0.2032) (layer F.Cu) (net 2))
 (segment (start 168.172595 86.995) (end 168.744095 87.5665) (width 0.2032) (layer F.Cu) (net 2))
 (segment (start 168.744095 87.5665) (end 170.819419 87.5665) (width 0.2032) (layer F.Cu) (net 2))
 (via (at 164.0586 87.0204) (size 0.508) (drill 0.254) (layers F.Cu B.Cu) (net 2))
 (segment (start 164.084 86.995) (end 164.0586 87.0204) (width 0.2032) (layer F.Cu) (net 2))
 (segment (start 167.0685 86.995) (end 164.084 86.995) (width 0.2032) (layer F.Cu) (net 2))
 (segment (start 162.5854 87.0204) (end 162.56 86.995) (width 0.2032) (layer B.Cu) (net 2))
 (segment (start 164.0586 87.0204) (end 162.5854 87.0204) (width 0.2032) (layer B.Cu) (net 2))
 (segment (start 160.592 86.995) (end 160.4772 87.1098) (width 0.2032) (layer B.Cu) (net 2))
 (segment (start 162.56 86.995) (end 160.592 86.995) (width 0.2032) (layer B.Cu) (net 2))
 (via (at 164.125002 83.756218) (size 0.508) (drill 0.254) (layers F.Cu B.Cu) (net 10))
 (segment (start 167.0685 84.455) (end 166.369718 83.756218) (width 0.2032) (layer F.Cu) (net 10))
 (segment (start 164.484212 83.756218) (end 164.125002 83.756218) (width 0.2032) (layer F.Cu) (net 10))
 (segment (start 166.369718 83.756218) (end 164.484212 83.756218) (width 0.2032) (layer F.Cu) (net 10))
 (segment (start 176.251501 84.176501) (end 177.1015 85.0265) (width 0.2032) (layer F.Cu) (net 10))
 (segment (start 175.84349 83.76849) (end 176.251501 84.176501) (width 0.2032) (layer F.Cu) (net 10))
 (segment (start 168.1435 84.455) (end 168.45391 84.76541) (width 0.2032) (layer F.Cu) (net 10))
 (segment (start 167.0685 84.455) (end 168.1435 84.455) (width 0.2032) (layer F.Cu) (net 10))
 (segment (start 168.45391 84.76541) (end 170.573484 84.76541) (width 0.2032) (layer F.Cu) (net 10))
 (segment (start 170.573484 84.76541) (end 171.570404 83.76849) (width 0.2032) (layer F.Cu) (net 10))
 (segment (start 171.570404 83.76849) (end 175.84349 83.76849) (width 0.2032) (layer F.Cu) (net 10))
 (segment (start 161.709587 83.756218) (end 161.22649 84.239315) (width 0.2032) (layer B.Cu) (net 10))
 (segment (start 161.22649 84.79791) (end 160.4772 85.5472) (width 0.2032) (layer B.Cu) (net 10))
 (segment (start 161.22649 84.239315) (end 161.22649 84.79791) (width 0.2032) (layer B.Cu) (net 10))
 (segment (start 164.125002 83.756218) (end 161.709587 83.756218) (width 0.2032) (layer B.Cu) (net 10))
 (segment (start 158.01652 88.25992) (end 156.94152 88.25992) (width 0.2032) (layer B.Cu) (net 10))
 (segment (start 158.24959 88.02685) (end 158.01652 88.25992) (width 0.2032) (layer B.Cu) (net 10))
 (segment (start 158.24959 86.732824) (end 158.24959 88.02685) (width 0.2032) (layer B.Cu) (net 10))
 (segment (start 158.743504 86.23891) (end 158.24959 86.732824) (width 0.2032) (layer B.Cu) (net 10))
 (segment (start 159.78549 86.23891) (end 158.743504 86.23891) (width 0.2032) (layer B.Cu) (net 10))
 (segment (start 160.4772 85.5472) (end 159.78549 86.23891) (width 0.2032) (layer B.Cu) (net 10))
 (segment (start 169.4688 85.5981) (end 168.711849 85.5981) (width 0.2032) (layer F.Cu) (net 11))
 (segment (start 168.711849 85.5981) (end 168.193759 85.08001) (width 0.2032) (layer F.Cu) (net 11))
 (segment (start 163.1935 84.455) (end 162.1185 84.455) (width 0.2032) (layer F.Cu) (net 11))
 (segment (start 164.624596 84.455) (end 163.1935 84.455) (width 0.2032) (layer F.Cu) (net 11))
 (segment (start 165.249606 85.08001) (end 164.624596 84.455) (width 0.2032) (layer F.Cu) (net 11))
 (segment (start 168.193759 85.08001) (end 165.249606 85.08001) (width 0.2032) (layer F.Cu) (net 11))
 (segment (start 157.22092 85.71992) (end 157.8102 86.3092) (width 0.2032) (layer B.Cu) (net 11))
 (via (at 157.8102 86.3092) (size 0.508) (drill 0.254) (layers F.Cu B.Cu) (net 11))
 (segment (start 156.94152 85.71992) (end 157.22092 85.71992) (width 0.2032) (layer B.Cu) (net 11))
 (segment (start 160.706586 84.455) (end 162.1185 84.455) (width 0.2032) (layer F.Cu) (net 11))
 (segment (start 158.852386 86.3092) (end 160.706586 84.455) (width 0.2032) (layer F.Cu) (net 11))
 (segment (start 157.8102 86.3092) (end 158.852386 86.3092) (width 0.2032) (layer F.Cu) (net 11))
 (segment (start 157.12948 86.98992) (end 157.8102 86.3092) (width 0.2032) (layer B.Cu) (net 11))
 (segment (start 156.94152 86.98992) (end 157.12948 86.98992) (width 0.2032) (layer B.Cu) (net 11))
 (via (at 153.2382 86.4616) (size 0.508) (drill 0.254) (layers F.Cu B.Cu) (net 8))
 (segment (start 152.70988 86.98992) (end 153.2382 86.4616) (width 0.2032) (layer B.Cu) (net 8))
 (segment (start 151.99152 86.98992) (end 152.70988 86.98992) (width 0.2032) (layer B.Cu) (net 8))
 (segment (start 149.627921 83.985999) (end 150.406899 84.764977) (width 0.2032) (layer B.Cu) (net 8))
 (segment (start 151.715162 86.98992) (end 151.99152 86.98992) (width 0.2032) (layer B.Cu) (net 8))
 (segment (start 148.568079 83.985999) (end 149.627921 83.985999) (width 0.2032) (layer B.Cu) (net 8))
 (segment (start 150.406899 84.764977) (end 150.406899 85.681657) (width 0.2032) (layer B.Cu) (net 8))
 (segment (start 147.993999 86.194001) (end 147.993999 84.560079) (width 0.2032) (layer B.Cu) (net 8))
 (segment (start 147.993999 84.560079) (end 148.568079 83.985999) (width 0.2032) (layer B.Cu) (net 8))
 (segment (start 146.558 87.63) (end 147.993999 86.194001) (width 0.2032) (layer B.Cu) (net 8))
 (segment (start 150.406899 85.681657) (end 151.715162 86.98992) (width 0.2032) (layer B.Cu) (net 8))
 (segment (start 153.2382 86.4616) (end 153.690988 86.008812) (width 0.2032) (layer F.Cu) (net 8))
 (segment (start 153.690988 86.008812) (end 156.408788 86.008812) (width 0.2032) (layer F.Cu) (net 8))
 (segment (start 156.408788 86.008812) (end 156.8704 85.5472) (width 0.2032) (layer F.Cu) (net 8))
 (segment (start 151.99152 85.71992) (end 151.361842 85.71992) (width 0.2032) (layer B.Cu) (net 7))
 (segment (start 146.558 85.09) (end 148.017612 83.630388) (width 0.2032) (layer B.Cu) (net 7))
 (segment (start 149.775219 83.630388) (end 150.76251 84.617679) (width 0.2032) (layer B.Cu) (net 7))
 (segment (start 148.017612 83.630388) (end 149.775219 83.630388) (width 0.2032) (layer B.Cu) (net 7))
 (segment (start 150.76251 84.617679) (end 150.76251 85.46591) (width 0.2032) (layer B.Cu) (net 7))
 (segment (start 150.76251 85.46591) (end 151.01652 85.71992) (width 0.2032) (layer B.Cu) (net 7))
 (segment (start 151.01652 85.71992) (end 151.99152 85.71992) (width 0.2032) (layer B.Cu) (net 7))
 (segment (start 151.99152 85.71992) (end 153.156767 85.71992) (width 0.2032) (layer B.Cu) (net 7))
 (segment (start 153.156767 85.71992) (end 153.209106 85.772259) (width 0.2032) (layer B.Cu) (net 7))
 (via (at 153.209106 85.772259) (size 0.508) (drill 0.254) (layers F.Cu B.Cu) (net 7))
 (segment (start 155.189399 85.653201) (end 156.8704 83.9722) (width 0.2032) (layer F.Cu) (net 7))
 (segment (start 153.328164 85.653201) (end 153.209106 85.772259) (width 0.2032) (layer F.Cu) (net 7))
 (segment (start 155.189399 85.653201) (end 153.328164 85.653201) (width 0.2032) (layer F.Cu) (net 7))
 (segment (start 170.49558 86.86851) (end 171.009599 86.354491) (width 0.2032) (layer F.Cu) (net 16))
 (segment (start 173.233509 86.354491) (end 173.711501 85.876499) (width 0.2032) (layer F.Cu) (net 16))
 (segment (start 173.711501 85.876499) (end 174.5615 85.0265) (width 0.2032) (layer F.Cu) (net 16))
 (segment (start 171.009599 86.354491) (end 173.233509 86.354491) (width 0.2032) (layer F.Cu) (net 16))
 (segment (start 168.682516 86.86851) (end 170.49558 86.86851) (width 0.2032) (layer F.Cu) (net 16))
 (segment (start 167.909716 86.09571) (end 168.682516 86.86851) (width 0.2032) (layer F.Cu) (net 16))
 (segment (start 167.0685 85.725) (end 167.43921 86.09571) (width 0.2032) (layer F.Cu) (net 16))
 (segment (start 167.43921 86.09571) (end 167.909716 86.09571) (width 0.2032) (layer F.Cu) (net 16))
 (via (at 168.8084 83.7946) (size 0.508) (drill 0.254) (layers F.Cu B.Cu) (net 15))
 (segment (start 169.1893 84.1755) (end 168.8084 83.7946) (width 0.2032) (layer B.Cu) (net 15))
 (segment (start 169.4815 84.1755) (end 169.1893 84.1755) (width 0.2032) (layer B.Cu) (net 15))
 (segment (start 169.0369 84.0231) (end 168.8084 83.7946) (width 0.2032) (layer F.Cu) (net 15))
 (segment (start 169.4688 84.0231) (end 169.0369 84.0231) (width 0.2032) (layer F.Cu) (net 15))
 (segment (start 158.9786 85.5474) (end 158.9786 85.2678) (width 0.2032) (layer B.Cu) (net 6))
 (segment (start 158.6484 85.3696) (end 158.4706 85.5474) (width 0.2032) (layer F.Cu) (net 6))
 (segment (start 158.6484 84.9376) (end 158.6484 85.3696) (width 0.2032) (layer F.Cu) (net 6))
 (segment (start 160.477 83.9724) (end 160.4772 83.9722) (width 0.2032) (layer B.Cu) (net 5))
 (segment (start 158.9786 85.2678) (end 158.6484 84.9376) (width 0.2032) (layer B.Cu) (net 6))
 (via (at 158.6484 84.9376) (size 0.508) (drill 0.254) (layers F.Cu B.Cu) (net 6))
 (segment (start 158.9788 83.9722) (end 158.9786 83.9724) (width 0.2032) (layer B.Cu) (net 5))
 (segment (start 160.4772 83.9722) (end 158.9788 83.9722) (width 0.2032) (layer B.Cu) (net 5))
 (segment (start 158.9786 83.9724) (end 158.50108 84.44992) (width 0.2032) (layer B.Cu) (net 5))
 (segment (start 158.50108 84.44992) (end 156.94152 84.44992) (width 0.2032) (layer B.Cu) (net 5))
 (segment (start 165.5976 86.995) (end 165.4048 87.1878) (width 0.2032) (layer B.Cu) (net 3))
 (segment (start 167.51 86.995) (end 165.5976 86.995) (width 0.2032) (layer B.Cu) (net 3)))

